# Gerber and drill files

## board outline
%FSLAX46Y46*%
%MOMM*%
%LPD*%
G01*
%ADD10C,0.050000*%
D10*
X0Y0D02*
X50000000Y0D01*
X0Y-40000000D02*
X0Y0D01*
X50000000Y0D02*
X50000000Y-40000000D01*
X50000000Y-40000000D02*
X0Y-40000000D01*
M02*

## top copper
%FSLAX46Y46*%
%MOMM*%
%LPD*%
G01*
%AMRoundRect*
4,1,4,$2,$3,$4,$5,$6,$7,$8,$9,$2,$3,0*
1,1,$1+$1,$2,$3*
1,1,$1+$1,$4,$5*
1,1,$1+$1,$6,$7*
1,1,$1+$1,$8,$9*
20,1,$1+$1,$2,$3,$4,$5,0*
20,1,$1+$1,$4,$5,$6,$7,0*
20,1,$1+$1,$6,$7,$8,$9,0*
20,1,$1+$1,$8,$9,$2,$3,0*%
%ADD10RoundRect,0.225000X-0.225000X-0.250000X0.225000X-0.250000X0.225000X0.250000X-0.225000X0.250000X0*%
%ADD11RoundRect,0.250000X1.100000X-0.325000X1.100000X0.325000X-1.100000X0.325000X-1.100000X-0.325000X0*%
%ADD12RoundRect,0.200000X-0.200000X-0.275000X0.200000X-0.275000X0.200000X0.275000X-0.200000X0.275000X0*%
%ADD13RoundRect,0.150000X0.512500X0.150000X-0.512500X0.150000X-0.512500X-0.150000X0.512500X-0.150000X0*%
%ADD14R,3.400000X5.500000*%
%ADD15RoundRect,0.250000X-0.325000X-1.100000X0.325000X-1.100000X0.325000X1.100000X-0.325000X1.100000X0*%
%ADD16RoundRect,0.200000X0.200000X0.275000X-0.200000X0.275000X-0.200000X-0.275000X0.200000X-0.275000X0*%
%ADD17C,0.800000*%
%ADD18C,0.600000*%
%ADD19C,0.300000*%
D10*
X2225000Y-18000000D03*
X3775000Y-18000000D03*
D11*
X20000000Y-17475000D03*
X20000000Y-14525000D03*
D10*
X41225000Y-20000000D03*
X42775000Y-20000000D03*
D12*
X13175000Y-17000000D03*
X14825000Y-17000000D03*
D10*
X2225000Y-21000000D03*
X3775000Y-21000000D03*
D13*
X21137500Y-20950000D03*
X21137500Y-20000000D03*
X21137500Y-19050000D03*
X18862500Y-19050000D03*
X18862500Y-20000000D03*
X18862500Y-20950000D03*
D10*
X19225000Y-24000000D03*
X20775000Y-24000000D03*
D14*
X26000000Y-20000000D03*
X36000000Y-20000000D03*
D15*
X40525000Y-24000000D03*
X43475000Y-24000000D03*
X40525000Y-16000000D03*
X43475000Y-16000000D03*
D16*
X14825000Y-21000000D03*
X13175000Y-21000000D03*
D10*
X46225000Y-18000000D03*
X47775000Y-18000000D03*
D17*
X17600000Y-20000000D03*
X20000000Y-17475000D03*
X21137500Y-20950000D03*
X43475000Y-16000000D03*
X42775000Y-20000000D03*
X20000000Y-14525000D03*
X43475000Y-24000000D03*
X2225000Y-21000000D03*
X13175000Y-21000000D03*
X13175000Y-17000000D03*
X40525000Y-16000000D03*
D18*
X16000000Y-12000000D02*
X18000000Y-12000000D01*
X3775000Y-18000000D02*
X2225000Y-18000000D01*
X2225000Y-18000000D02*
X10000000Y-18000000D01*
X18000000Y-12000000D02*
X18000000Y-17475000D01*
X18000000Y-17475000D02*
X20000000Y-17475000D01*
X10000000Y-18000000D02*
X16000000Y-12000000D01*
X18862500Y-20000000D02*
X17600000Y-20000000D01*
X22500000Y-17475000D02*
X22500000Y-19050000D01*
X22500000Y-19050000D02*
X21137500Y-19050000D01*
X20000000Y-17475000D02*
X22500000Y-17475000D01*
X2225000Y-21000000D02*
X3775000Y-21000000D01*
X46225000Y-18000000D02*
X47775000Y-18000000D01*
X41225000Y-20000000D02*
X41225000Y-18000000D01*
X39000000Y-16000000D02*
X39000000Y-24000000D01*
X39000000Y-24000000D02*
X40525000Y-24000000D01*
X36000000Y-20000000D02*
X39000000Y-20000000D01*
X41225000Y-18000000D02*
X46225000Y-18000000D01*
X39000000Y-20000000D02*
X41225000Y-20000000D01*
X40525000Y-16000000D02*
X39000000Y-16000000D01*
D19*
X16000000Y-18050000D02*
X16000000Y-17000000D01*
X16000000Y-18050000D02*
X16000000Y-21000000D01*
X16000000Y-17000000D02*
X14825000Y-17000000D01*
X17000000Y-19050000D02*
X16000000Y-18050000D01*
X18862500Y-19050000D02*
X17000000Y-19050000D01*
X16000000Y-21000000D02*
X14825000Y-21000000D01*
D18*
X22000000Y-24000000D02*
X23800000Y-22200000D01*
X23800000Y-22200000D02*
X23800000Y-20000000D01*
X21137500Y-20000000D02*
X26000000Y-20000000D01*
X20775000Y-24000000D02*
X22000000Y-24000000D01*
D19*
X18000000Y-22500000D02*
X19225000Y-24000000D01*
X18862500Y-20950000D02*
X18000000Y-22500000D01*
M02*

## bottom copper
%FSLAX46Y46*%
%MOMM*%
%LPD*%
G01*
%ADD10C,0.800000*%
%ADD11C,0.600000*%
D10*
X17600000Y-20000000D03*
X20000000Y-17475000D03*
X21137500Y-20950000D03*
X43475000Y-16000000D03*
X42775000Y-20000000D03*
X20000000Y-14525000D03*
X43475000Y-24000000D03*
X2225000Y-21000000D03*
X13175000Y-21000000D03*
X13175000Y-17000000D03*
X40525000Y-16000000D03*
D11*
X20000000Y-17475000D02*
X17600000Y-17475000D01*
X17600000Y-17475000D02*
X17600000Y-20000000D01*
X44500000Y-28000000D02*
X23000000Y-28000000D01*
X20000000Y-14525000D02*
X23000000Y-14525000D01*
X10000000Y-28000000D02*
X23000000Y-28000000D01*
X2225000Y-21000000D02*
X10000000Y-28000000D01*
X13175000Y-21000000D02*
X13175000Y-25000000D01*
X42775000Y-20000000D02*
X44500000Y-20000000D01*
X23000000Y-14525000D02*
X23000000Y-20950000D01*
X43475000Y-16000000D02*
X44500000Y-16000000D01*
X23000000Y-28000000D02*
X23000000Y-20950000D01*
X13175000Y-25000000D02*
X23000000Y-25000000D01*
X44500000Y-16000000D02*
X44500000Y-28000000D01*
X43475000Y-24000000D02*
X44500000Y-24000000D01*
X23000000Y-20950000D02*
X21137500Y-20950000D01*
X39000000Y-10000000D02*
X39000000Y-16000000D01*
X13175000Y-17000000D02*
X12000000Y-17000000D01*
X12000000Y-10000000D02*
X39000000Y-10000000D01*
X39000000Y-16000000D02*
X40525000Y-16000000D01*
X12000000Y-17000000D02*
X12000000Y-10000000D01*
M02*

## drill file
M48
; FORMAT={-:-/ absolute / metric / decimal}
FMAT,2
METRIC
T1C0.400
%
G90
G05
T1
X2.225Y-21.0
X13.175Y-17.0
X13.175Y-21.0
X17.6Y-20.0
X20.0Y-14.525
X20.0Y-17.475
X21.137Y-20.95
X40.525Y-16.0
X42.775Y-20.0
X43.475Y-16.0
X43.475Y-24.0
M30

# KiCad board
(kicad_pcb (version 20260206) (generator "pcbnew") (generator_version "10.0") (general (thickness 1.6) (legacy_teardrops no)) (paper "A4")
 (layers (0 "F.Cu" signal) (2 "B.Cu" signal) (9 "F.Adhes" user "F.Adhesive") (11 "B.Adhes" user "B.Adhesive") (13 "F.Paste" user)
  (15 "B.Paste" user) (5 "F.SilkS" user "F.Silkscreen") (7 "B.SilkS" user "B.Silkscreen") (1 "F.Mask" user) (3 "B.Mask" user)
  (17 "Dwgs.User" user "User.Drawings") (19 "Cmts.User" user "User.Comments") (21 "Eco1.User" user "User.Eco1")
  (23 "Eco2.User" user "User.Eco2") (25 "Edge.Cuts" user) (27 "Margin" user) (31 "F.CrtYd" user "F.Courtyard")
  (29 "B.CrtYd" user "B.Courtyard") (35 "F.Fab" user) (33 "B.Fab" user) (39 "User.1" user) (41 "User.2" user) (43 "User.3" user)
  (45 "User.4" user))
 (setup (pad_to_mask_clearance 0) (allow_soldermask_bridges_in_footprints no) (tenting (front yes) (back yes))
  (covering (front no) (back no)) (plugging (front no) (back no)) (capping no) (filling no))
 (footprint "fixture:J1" (layer "F.Cu") (at 3 18)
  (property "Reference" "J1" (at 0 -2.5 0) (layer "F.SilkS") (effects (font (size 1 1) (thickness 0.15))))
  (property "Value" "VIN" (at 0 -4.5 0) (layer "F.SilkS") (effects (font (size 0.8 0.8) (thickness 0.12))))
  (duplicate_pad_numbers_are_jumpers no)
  (pad "1" smd roundrect (at -0.775 0) (size 0.9 0.95) (layers "F.Cu" "F.Mask" "F.Paste") (roundrect_rratio 0.25) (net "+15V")
   (thermal_bridge_angle 45))
  (pad "2" smd roundrect (at 0.775 0) (size 0.9 0.95) (layers "F.Cu" "F.Mask" "F.Paste") (roundrect_rratio 0.25) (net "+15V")
   (thermal_bridge_angle 45)))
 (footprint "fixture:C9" (layer "F.Cu") (at 20 16 90)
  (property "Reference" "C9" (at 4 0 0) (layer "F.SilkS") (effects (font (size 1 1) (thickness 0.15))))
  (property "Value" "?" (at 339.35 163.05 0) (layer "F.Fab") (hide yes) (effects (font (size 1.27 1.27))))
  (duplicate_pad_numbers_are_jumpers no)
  (pad "1" smd roundrect (at -1.475 0 90) (size 1.15 2.7) (layers "F.Cu" "F.Mask" "F.Paste") (roundrect_rratio 0.217391) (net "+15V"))
  (pad "2" smd roundrect (at 1.475 0 90) (size 1.15 2.7) (layers "F.Cu" "F.Mask" "F.Paste") (roundrect_rratio 0.217391) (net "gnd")))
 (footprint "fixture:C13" (layer "F.Cu") (at 42 20)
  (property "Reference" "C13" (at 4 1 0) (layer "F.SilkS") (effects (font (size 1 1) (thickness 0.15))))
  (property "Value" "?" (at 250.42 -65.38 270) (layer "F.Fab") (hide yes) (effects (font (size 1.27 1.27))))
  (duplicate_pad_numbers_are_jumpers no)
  (pad "1" smd roundrect (at -0.775 0) (size 0.9 0.95) (layers "F.Cu" "F.Mask" "F.Paste") (roundrect_rratio 0.25) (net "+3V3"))
  (pad "2" smd roundrect (at 0.775 0) (size 0.9 0.95) (layers "F.Cu" "F.Mask" "F.Paste") (roundrect_rratio 0.25) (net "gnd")))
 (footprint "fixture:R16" (layer "F.Cu") (at 14 17)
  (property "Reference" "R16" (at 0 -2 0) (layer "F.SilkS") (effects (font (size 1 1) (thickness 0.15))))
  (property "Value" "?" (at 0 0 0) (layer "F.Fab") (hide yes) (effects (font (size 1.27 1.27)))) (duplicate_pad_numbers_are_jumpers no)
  (pad "1" smd roundrect (at -0.825 0) (size 0.8 0.95) (layers "F.Cu" "F.Mask" "F.Paste") (roundrect_rratio 0.25) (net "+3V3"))
  (pad "2" smd roundrect (at 0.825 0) (size 0.8 0.95) (layers "F.Cu" "F.Mask" "F.Paste") (roundrect_rratio 0.25) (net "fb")))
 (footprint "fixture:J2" (layer "F.Cu") (at 3 21)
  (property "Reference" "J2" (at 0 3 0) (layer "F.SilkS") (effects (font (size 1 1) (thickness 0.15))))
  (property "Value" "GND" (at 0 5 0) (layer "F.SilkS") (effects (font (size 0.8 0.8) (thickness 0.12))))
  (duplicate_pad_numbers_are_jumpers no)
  (pad "1" smd roundrect (at -0.775 0) (size 0.9 0.95) (layers "F.Cu" "F.Mask" "F.Paste") (roundrect_rratio 0.25) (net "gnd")
   (thermal_bridge_angle 45))
  (pad "2" smd roundrect (at 0.775 0) (size 0.9 0.95) (layers "F.Cu" "F.Mask" "F.Paste") (roundrect_rratio 0.25) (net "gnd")
   (thermal_bridge_angle 45)))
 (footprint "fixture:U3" (layer "F.Cu") (at 20 20 180)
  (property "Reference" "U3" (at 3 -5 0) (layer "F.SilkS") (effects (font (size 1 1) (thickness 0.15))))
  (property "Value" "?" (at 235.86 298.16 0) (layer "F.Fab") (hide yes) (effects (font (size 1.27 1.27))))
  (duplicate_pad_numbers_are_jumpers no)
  (pad "1" smd roundrect (at -1.1375 -0.95 180) (size 1.325 0.6) (layers "F.Cu" "F.Mask" "F.Paste") (roundrect_rratio 0.25) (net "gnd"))
  (pad "2" smd roundrect (at -1.1375 0 180) (size 1.325 0.6) (layers "F.Cu" "F.Mask" "F.Paste") (roundrect_rratio 0.25) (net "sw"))
  (pad "3" smd roundrect (at -1.1375 0.95 180) (size 1.325 0.6) (layers "F.Cu" "F.Mask" "F.Paste") (roundrect_rratio 0.25) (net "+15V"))
  (pad "4" smd roundrect (at 1.1375 0.95 180) (size 1.325 0.6) (layers "F.Cu" "F.Mask" "F.Paste") (roundrect_rratio 0.25) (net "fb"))
  (pad "5" smd roundrect (at 1.1375 0 180) (size 1.325 0.6) (layers "F.Cu" "F.Mask" "F.Paste") (roundrect_rratio 0.25) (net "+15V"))
  (pad "6" smd roundrect (at 1.1375 -0.95 180) (size 1.325 0.6) (layers "F.Cu" "F.Mask" "F.Paste") (roundrect_rratio 0.25) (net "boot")))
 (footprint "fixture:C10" (layer "F.Cu") (at 20 24)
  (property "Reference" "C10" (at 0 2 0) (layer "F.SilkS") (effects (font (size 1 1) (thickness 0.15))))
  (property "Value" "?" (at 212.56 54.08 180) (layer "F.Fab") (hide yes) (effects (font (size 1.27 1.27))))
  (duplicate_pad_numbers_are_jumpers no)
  (pad "1" smd roundrect (at -0.775 0) (size 0.9 0.95) (layers "F.Cu" "F.Mask" "F.Paste") (roundrect_rratio 0.25) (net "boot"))
  (pad "2" smd roundrect (at 0.775 0) (size 0.9 0.95) (layers "F.Cu" "F.Mask" "F.Paste") (roundrect_rratio 0.25) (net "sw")))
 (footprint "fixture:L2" (layer "F.Cu") (at 31 20)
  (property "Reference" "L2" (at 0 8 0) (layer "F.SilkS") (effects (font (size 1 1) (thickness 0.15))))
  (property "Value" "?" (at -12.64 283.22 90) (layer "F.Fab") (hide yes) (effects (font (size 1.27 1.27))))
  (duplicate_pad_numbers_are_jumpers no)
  (pad "1" smd rect (at -5 0) (size 3.4 5.5) (layers "F.Cu" "F.Mask" "F.Paste") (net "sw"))
  (pad "2" smd rect (at 5 0) (size 3.4 5.5) (layers "F.Cu" "F.Mask" "F.Paste") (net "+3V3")))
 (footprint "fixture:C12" (layer "F.Cu") (at 42 24)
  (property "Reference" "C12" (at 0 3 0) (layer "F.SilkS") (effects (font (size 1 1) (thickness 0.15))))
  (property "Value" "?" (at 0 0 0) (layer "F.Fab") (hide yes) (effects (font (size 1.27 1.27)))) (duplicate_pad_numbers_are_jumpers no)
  (pad "1" smd roundrect (at -1.475 0) (size 1.15 2.7) (layers "F.Cu" "F.Mask" "F.Paste") (roundrect_rratio 0.217391) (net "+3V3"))
  (pad "2" smd roundrect (at 1.475 0) (size 1.15 2.7) (layers "F.Cu" "F.Mask" "F.Paste") (roundrect_rratio 0.217391) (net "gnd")))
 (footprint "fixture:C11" (layer "F.Cu") (at 42 16)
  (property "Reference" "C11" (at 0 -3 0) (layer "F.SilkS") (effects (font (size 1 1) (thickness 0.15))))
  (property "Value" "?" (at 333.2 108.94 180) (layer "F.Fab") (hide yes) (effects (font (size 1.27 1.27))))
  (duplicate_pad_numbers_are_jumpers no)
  (pad "1" smd roundrect (at -1.475 0) (size 1.15 2.7) (layers "F.Cu" "F.Mask" "F.Paste") (roundrect_rratio 0.217391) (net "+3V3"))
  (pad "2" smd roundrect (at 1.475 0) (size 1.15 2.7) (layers "F.Cu" "F.Mask" "F.Paste") (roundrect_rratio 0.217391) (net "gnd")))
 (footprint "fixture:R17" (layer "F.Cu") (at 14 21 180)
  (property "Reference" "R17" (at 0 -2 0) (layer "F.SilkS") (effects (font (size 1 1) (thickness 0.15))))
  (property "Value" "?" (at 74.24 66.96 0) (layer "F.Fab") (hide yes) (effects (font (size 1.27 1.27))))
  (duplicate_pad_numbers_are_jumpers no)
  (pad "1" smd roundrect (at -0.825 0 180) (size 0.8 0.95) (layers "F.Cu" "F.Mask" "F.Paste") (roundrect_rratio 0.25) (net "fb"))
  (pad "2" smd roundrect (at 0.825 0 180) (size 0.8 0.95) (layers "F.Cu" "F.Mask" "F.Paste") (roundrect_rratio 0.25) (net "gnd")))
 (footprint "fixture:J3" (layer "F.Cu") (at 47 18)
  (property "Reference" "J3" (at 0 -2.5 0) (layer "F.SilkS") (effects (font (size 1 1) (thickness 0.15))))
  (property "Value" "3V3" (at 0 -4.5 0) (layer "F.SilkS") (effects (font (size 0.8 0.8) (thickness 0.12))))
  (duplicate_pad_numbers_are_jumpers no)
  (pad "1" smd roundrect (at -0.775 0) (size 0.9 0.95) (layers "F.Cu" "F.Mask" "F.Paste") (roundrect_rratio 0.25) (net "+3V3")
   (thermal_bridge_angle 45))
  (pad "2" smd roundrect (at 0.775 0) (size 0.9 0.95) (layers "F.Cu" "F.Mask" "F.Paste") (roundrect_rratio 0.25) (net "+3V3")
   (thermal_bridge_angle 45)))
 (gr_line (start 0 0) (end 50 0) (stroke (width 0.05) (type default)) (layer "Edge.Cuts"))
 (gr_line (start 0 40) (end 0 0) (stroke (width 0.05) (type default)) (layer "Edge.Cuts"))
 (gr_line (start 50 0) (end 50 40) (stroke (width 0.05) (type default)) (layer "Edge.Cuts"))
 (gr_line (start 50 40) (end 0 40) (stroke (width 0.05) (type default)) (layer "Edge.Cuts"))
 (segment (start 16 12) (end 18 12) (width 0.6) (layer "F.Cu") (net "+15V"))
 (segment (start 3.775 18) (end 2.225 18) (width 0.6) (layer "F.Cu") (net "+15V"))
 (segment (start 2.225 18) (end 10 18) (width 0.6) (layer "F.Cu") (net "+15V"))
 (segment (start 18 12) (end 18 17.475) (width 0.6) (layer "F.Cu") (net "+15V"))
 (segment (start 18 17.475) (end 20 17.475) (width 0.6) (layer "F.Cu") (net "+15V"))
 (segment (start 10 18) (end 16 12) (width 0.6) (layer "F.Cu") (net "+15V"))
 (segment (start 18.8625 20) (end 17.6 20) (width 0.6) (layer "F.Cu") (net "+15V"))
 (segment (start 22.5 17.475) (end 22.5 19.05) (width 0.6) (layer "F.Cu") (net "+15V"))
 (segment (start 22.5 19.05) (end 21.1375 19.05) (width 0.6) (layer "F.Cu") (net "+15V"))
 (segment (start 20 17.475) (end 22.5 17.475) (width 0.6) (layer "F.Cu") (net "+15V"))
 (via (at 17.6 20) (size 0.8) (drill 0.4) (layers "F.Cu" "B.Cu") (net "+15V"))
 (via (at 20 17.475) (size 0.8) (drill 0.4) (layers "F.Cu" "B.Cu") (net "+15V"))
 (segment (start 20 17.475) (end 17.6 17.475) (width 0.6) (layer "B.Cu") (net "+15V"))
 (segment (start 17.6 17.475) (end 17.6 20) (width 0.6) (layer "B.Cu") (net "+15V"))
 (segment (start 2.225 21) (end 3.775 21) (width 0.6) (layer "F.Cu") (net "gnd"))
 (via (at 21.1375 20.95) (size 0.8) (drill 0.4) (layers "F.Cu" "B.Cu") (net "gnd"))
 (via (at 43.475 16) (size 0.8) (drill 0.4) (layers "F.Cu" "B.Cu") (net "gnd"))
 (via (at 42.775 20) (size 0.8) (drill 0.4) (layers "F.Cu" "B.Cu") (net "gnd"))
 (via (at 20 14.525) (size 0.8) (drill 0.4) (layers "F.Cu" "B.Cu") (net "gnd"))
 (via (at 43.475 24) (size 0.8) (drill 0.4) (layers "F.Cu" "B.Cu") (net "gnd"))
 (via (at 2.225 21) (size 0.8) (drill 0.4) (layers "F.Cu" "B.Cu") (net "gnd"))
 (via (at 13.175 21) (size 0.8) (drill 0.4) (layers "F.Cu" "B.Cu") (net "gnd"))
 (segment (start 44.5 28) (end 23 28) (width 0.6) (layer "B.Cu") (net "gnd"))
 (segment (start 20 14.525) (end 23 14.525) (width 0.6) (layer "B.Cu") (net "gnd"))
 (segment (start 10 28) (end 23 28) (width 0.6) (layer "B.Cu") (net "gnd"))
 (segment (start 2.225 21) (end 10 28) (width 0.6) (layer "B.Cu") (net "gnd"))
 (segment (start 13.175 21) (end 13.175 25) (width 0.6) (layer "B.Cu") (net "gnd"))
 (segment (start 42.775 20) (end 44.5 20) (width 0.6) (layer "B.Cu") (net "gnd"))
 (segment (start 23 14.525) (end 23 20.95) (width 0.6) (layer "B.Cu") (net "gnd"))
 (segment (start 43.475 16) (end 44.5 16) (width 0.6) (layer "B.Cu") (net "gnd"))
 (segment (start 23 28) (end 23 20.95) (width 0.6) (layer "B.Cu") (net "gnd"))
 (segment (start 13.175 25) (end 23 25) (width 0.6) (layer "B.Cu") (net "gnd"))
 (segment (start 44.5 16) (end 44.5 28) (width 0.6) (layer "B.Cu") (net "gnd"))
 (segment (start 43.475 24) (end 44.5 24) (width 0.6) (layer "B.Cu") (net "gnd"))
 (segment (start 23 20.95) (end 21.1375 20.95) (width 0.6) (layer "B.Cu") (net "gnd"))
 (segment (start 46.225 18) (end 47.775 18) (width 0.6) (layer "F.Cu") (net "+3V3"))
 (segment (start 41.225 20) (end 41.225 18) (width 0.6) (layer "F.Cu") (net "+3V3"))
 (segment (start 39 16) (end 39 24) (width 0.6) (layer "F.Cu") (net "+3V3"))
 (segment (start 39 24) (end 40.525 24) (width 0.6) (layer "F.Cu") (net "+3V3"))
 (segment (start 36 20) (end 39 20) (width 0.6) (layer "F.Cu") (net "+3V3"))
 (segment (start 41.225 18) (end 46.225 18) (width 0.6) (layer "F.Cu") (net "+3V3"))
 (segment (start 39 20) (end 41.225 20) (width 0.6) (layer "F.Cu") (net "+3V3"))
 (segment (start 40.525 16) (end 39 16) (width 0.6) (layer "F.Cu") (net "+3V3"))
 (via (at 13.175 17) (size 0.8) (drill 0.4) (layers "F.Cu" "B.Cu") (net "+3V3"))
 (via (at 40.525 16) (size 0.8) (drill 0.4) (layers "F.Cu" "B.Cu") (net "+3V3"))
 (segment (start 39 10) (end 39 16) (width 0.6) (layer "B.Cu") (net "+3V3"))
 (segment (start 13.175 17) (end 12 17) (width 0.6) (layer "B.Cu") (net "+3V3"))
 (segment (start 12 10) (end 39 10) (width 0.6) (layer "B.Cu") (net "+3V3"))
 (segment (start 39 16) (end 40.525 16) (width 0.6) (layer "B.Cu") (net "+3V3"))
 (segment (start 12 17) (end 12 10) (width 0.6) (layer "B.Cu") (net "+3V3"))
 (segment (start 16 18.05) (end 16 17) (width 0.3) (layer "F.Cu") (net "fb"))
 (segment (start 16 18.05) (end 16 21) (width 0.3) (layer "F.Cu") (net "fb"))
 (segment (start 16 17) (end 14.825 17) (width 0.3) (layer "F.Cu") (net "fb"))
 (segment (start 17 19.05) (end 16 18.05) (width 0.3) (layer "F.Cu") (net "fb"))
 (segment (start 18.8625 19.05) (end 17 19.05) (width 0.3) (layer "F.Cu") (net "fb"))
 (segment (start 16 21) (end 14.825 21) (width 0.3) (layer "F.Cu") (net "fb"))
 (segment (start 22 24) (end 23.8 22.2) (width 0.6) (layer "F.Cu") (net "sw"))
 (segment (start 23.8 22.2) (end 23.8 20) (width 0.6) (layer "F.Cu") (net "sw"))
 (segment (start 21.1375 20) (end 26 20) (width 0.6) (layer "F.Cu") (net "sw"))
 (segment (start 20.775 24) (end 22 24) (width 0.6) (layer "F.Cu") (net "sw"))
 (segment (start 18 22.5) (end 19.225 24) (width 0.3) (layer "F.Cu") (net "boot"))
 (segment (start 18.8625 20.95) (end 18 22.5) (width 0.3) (layer "F.Cu") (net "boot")))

